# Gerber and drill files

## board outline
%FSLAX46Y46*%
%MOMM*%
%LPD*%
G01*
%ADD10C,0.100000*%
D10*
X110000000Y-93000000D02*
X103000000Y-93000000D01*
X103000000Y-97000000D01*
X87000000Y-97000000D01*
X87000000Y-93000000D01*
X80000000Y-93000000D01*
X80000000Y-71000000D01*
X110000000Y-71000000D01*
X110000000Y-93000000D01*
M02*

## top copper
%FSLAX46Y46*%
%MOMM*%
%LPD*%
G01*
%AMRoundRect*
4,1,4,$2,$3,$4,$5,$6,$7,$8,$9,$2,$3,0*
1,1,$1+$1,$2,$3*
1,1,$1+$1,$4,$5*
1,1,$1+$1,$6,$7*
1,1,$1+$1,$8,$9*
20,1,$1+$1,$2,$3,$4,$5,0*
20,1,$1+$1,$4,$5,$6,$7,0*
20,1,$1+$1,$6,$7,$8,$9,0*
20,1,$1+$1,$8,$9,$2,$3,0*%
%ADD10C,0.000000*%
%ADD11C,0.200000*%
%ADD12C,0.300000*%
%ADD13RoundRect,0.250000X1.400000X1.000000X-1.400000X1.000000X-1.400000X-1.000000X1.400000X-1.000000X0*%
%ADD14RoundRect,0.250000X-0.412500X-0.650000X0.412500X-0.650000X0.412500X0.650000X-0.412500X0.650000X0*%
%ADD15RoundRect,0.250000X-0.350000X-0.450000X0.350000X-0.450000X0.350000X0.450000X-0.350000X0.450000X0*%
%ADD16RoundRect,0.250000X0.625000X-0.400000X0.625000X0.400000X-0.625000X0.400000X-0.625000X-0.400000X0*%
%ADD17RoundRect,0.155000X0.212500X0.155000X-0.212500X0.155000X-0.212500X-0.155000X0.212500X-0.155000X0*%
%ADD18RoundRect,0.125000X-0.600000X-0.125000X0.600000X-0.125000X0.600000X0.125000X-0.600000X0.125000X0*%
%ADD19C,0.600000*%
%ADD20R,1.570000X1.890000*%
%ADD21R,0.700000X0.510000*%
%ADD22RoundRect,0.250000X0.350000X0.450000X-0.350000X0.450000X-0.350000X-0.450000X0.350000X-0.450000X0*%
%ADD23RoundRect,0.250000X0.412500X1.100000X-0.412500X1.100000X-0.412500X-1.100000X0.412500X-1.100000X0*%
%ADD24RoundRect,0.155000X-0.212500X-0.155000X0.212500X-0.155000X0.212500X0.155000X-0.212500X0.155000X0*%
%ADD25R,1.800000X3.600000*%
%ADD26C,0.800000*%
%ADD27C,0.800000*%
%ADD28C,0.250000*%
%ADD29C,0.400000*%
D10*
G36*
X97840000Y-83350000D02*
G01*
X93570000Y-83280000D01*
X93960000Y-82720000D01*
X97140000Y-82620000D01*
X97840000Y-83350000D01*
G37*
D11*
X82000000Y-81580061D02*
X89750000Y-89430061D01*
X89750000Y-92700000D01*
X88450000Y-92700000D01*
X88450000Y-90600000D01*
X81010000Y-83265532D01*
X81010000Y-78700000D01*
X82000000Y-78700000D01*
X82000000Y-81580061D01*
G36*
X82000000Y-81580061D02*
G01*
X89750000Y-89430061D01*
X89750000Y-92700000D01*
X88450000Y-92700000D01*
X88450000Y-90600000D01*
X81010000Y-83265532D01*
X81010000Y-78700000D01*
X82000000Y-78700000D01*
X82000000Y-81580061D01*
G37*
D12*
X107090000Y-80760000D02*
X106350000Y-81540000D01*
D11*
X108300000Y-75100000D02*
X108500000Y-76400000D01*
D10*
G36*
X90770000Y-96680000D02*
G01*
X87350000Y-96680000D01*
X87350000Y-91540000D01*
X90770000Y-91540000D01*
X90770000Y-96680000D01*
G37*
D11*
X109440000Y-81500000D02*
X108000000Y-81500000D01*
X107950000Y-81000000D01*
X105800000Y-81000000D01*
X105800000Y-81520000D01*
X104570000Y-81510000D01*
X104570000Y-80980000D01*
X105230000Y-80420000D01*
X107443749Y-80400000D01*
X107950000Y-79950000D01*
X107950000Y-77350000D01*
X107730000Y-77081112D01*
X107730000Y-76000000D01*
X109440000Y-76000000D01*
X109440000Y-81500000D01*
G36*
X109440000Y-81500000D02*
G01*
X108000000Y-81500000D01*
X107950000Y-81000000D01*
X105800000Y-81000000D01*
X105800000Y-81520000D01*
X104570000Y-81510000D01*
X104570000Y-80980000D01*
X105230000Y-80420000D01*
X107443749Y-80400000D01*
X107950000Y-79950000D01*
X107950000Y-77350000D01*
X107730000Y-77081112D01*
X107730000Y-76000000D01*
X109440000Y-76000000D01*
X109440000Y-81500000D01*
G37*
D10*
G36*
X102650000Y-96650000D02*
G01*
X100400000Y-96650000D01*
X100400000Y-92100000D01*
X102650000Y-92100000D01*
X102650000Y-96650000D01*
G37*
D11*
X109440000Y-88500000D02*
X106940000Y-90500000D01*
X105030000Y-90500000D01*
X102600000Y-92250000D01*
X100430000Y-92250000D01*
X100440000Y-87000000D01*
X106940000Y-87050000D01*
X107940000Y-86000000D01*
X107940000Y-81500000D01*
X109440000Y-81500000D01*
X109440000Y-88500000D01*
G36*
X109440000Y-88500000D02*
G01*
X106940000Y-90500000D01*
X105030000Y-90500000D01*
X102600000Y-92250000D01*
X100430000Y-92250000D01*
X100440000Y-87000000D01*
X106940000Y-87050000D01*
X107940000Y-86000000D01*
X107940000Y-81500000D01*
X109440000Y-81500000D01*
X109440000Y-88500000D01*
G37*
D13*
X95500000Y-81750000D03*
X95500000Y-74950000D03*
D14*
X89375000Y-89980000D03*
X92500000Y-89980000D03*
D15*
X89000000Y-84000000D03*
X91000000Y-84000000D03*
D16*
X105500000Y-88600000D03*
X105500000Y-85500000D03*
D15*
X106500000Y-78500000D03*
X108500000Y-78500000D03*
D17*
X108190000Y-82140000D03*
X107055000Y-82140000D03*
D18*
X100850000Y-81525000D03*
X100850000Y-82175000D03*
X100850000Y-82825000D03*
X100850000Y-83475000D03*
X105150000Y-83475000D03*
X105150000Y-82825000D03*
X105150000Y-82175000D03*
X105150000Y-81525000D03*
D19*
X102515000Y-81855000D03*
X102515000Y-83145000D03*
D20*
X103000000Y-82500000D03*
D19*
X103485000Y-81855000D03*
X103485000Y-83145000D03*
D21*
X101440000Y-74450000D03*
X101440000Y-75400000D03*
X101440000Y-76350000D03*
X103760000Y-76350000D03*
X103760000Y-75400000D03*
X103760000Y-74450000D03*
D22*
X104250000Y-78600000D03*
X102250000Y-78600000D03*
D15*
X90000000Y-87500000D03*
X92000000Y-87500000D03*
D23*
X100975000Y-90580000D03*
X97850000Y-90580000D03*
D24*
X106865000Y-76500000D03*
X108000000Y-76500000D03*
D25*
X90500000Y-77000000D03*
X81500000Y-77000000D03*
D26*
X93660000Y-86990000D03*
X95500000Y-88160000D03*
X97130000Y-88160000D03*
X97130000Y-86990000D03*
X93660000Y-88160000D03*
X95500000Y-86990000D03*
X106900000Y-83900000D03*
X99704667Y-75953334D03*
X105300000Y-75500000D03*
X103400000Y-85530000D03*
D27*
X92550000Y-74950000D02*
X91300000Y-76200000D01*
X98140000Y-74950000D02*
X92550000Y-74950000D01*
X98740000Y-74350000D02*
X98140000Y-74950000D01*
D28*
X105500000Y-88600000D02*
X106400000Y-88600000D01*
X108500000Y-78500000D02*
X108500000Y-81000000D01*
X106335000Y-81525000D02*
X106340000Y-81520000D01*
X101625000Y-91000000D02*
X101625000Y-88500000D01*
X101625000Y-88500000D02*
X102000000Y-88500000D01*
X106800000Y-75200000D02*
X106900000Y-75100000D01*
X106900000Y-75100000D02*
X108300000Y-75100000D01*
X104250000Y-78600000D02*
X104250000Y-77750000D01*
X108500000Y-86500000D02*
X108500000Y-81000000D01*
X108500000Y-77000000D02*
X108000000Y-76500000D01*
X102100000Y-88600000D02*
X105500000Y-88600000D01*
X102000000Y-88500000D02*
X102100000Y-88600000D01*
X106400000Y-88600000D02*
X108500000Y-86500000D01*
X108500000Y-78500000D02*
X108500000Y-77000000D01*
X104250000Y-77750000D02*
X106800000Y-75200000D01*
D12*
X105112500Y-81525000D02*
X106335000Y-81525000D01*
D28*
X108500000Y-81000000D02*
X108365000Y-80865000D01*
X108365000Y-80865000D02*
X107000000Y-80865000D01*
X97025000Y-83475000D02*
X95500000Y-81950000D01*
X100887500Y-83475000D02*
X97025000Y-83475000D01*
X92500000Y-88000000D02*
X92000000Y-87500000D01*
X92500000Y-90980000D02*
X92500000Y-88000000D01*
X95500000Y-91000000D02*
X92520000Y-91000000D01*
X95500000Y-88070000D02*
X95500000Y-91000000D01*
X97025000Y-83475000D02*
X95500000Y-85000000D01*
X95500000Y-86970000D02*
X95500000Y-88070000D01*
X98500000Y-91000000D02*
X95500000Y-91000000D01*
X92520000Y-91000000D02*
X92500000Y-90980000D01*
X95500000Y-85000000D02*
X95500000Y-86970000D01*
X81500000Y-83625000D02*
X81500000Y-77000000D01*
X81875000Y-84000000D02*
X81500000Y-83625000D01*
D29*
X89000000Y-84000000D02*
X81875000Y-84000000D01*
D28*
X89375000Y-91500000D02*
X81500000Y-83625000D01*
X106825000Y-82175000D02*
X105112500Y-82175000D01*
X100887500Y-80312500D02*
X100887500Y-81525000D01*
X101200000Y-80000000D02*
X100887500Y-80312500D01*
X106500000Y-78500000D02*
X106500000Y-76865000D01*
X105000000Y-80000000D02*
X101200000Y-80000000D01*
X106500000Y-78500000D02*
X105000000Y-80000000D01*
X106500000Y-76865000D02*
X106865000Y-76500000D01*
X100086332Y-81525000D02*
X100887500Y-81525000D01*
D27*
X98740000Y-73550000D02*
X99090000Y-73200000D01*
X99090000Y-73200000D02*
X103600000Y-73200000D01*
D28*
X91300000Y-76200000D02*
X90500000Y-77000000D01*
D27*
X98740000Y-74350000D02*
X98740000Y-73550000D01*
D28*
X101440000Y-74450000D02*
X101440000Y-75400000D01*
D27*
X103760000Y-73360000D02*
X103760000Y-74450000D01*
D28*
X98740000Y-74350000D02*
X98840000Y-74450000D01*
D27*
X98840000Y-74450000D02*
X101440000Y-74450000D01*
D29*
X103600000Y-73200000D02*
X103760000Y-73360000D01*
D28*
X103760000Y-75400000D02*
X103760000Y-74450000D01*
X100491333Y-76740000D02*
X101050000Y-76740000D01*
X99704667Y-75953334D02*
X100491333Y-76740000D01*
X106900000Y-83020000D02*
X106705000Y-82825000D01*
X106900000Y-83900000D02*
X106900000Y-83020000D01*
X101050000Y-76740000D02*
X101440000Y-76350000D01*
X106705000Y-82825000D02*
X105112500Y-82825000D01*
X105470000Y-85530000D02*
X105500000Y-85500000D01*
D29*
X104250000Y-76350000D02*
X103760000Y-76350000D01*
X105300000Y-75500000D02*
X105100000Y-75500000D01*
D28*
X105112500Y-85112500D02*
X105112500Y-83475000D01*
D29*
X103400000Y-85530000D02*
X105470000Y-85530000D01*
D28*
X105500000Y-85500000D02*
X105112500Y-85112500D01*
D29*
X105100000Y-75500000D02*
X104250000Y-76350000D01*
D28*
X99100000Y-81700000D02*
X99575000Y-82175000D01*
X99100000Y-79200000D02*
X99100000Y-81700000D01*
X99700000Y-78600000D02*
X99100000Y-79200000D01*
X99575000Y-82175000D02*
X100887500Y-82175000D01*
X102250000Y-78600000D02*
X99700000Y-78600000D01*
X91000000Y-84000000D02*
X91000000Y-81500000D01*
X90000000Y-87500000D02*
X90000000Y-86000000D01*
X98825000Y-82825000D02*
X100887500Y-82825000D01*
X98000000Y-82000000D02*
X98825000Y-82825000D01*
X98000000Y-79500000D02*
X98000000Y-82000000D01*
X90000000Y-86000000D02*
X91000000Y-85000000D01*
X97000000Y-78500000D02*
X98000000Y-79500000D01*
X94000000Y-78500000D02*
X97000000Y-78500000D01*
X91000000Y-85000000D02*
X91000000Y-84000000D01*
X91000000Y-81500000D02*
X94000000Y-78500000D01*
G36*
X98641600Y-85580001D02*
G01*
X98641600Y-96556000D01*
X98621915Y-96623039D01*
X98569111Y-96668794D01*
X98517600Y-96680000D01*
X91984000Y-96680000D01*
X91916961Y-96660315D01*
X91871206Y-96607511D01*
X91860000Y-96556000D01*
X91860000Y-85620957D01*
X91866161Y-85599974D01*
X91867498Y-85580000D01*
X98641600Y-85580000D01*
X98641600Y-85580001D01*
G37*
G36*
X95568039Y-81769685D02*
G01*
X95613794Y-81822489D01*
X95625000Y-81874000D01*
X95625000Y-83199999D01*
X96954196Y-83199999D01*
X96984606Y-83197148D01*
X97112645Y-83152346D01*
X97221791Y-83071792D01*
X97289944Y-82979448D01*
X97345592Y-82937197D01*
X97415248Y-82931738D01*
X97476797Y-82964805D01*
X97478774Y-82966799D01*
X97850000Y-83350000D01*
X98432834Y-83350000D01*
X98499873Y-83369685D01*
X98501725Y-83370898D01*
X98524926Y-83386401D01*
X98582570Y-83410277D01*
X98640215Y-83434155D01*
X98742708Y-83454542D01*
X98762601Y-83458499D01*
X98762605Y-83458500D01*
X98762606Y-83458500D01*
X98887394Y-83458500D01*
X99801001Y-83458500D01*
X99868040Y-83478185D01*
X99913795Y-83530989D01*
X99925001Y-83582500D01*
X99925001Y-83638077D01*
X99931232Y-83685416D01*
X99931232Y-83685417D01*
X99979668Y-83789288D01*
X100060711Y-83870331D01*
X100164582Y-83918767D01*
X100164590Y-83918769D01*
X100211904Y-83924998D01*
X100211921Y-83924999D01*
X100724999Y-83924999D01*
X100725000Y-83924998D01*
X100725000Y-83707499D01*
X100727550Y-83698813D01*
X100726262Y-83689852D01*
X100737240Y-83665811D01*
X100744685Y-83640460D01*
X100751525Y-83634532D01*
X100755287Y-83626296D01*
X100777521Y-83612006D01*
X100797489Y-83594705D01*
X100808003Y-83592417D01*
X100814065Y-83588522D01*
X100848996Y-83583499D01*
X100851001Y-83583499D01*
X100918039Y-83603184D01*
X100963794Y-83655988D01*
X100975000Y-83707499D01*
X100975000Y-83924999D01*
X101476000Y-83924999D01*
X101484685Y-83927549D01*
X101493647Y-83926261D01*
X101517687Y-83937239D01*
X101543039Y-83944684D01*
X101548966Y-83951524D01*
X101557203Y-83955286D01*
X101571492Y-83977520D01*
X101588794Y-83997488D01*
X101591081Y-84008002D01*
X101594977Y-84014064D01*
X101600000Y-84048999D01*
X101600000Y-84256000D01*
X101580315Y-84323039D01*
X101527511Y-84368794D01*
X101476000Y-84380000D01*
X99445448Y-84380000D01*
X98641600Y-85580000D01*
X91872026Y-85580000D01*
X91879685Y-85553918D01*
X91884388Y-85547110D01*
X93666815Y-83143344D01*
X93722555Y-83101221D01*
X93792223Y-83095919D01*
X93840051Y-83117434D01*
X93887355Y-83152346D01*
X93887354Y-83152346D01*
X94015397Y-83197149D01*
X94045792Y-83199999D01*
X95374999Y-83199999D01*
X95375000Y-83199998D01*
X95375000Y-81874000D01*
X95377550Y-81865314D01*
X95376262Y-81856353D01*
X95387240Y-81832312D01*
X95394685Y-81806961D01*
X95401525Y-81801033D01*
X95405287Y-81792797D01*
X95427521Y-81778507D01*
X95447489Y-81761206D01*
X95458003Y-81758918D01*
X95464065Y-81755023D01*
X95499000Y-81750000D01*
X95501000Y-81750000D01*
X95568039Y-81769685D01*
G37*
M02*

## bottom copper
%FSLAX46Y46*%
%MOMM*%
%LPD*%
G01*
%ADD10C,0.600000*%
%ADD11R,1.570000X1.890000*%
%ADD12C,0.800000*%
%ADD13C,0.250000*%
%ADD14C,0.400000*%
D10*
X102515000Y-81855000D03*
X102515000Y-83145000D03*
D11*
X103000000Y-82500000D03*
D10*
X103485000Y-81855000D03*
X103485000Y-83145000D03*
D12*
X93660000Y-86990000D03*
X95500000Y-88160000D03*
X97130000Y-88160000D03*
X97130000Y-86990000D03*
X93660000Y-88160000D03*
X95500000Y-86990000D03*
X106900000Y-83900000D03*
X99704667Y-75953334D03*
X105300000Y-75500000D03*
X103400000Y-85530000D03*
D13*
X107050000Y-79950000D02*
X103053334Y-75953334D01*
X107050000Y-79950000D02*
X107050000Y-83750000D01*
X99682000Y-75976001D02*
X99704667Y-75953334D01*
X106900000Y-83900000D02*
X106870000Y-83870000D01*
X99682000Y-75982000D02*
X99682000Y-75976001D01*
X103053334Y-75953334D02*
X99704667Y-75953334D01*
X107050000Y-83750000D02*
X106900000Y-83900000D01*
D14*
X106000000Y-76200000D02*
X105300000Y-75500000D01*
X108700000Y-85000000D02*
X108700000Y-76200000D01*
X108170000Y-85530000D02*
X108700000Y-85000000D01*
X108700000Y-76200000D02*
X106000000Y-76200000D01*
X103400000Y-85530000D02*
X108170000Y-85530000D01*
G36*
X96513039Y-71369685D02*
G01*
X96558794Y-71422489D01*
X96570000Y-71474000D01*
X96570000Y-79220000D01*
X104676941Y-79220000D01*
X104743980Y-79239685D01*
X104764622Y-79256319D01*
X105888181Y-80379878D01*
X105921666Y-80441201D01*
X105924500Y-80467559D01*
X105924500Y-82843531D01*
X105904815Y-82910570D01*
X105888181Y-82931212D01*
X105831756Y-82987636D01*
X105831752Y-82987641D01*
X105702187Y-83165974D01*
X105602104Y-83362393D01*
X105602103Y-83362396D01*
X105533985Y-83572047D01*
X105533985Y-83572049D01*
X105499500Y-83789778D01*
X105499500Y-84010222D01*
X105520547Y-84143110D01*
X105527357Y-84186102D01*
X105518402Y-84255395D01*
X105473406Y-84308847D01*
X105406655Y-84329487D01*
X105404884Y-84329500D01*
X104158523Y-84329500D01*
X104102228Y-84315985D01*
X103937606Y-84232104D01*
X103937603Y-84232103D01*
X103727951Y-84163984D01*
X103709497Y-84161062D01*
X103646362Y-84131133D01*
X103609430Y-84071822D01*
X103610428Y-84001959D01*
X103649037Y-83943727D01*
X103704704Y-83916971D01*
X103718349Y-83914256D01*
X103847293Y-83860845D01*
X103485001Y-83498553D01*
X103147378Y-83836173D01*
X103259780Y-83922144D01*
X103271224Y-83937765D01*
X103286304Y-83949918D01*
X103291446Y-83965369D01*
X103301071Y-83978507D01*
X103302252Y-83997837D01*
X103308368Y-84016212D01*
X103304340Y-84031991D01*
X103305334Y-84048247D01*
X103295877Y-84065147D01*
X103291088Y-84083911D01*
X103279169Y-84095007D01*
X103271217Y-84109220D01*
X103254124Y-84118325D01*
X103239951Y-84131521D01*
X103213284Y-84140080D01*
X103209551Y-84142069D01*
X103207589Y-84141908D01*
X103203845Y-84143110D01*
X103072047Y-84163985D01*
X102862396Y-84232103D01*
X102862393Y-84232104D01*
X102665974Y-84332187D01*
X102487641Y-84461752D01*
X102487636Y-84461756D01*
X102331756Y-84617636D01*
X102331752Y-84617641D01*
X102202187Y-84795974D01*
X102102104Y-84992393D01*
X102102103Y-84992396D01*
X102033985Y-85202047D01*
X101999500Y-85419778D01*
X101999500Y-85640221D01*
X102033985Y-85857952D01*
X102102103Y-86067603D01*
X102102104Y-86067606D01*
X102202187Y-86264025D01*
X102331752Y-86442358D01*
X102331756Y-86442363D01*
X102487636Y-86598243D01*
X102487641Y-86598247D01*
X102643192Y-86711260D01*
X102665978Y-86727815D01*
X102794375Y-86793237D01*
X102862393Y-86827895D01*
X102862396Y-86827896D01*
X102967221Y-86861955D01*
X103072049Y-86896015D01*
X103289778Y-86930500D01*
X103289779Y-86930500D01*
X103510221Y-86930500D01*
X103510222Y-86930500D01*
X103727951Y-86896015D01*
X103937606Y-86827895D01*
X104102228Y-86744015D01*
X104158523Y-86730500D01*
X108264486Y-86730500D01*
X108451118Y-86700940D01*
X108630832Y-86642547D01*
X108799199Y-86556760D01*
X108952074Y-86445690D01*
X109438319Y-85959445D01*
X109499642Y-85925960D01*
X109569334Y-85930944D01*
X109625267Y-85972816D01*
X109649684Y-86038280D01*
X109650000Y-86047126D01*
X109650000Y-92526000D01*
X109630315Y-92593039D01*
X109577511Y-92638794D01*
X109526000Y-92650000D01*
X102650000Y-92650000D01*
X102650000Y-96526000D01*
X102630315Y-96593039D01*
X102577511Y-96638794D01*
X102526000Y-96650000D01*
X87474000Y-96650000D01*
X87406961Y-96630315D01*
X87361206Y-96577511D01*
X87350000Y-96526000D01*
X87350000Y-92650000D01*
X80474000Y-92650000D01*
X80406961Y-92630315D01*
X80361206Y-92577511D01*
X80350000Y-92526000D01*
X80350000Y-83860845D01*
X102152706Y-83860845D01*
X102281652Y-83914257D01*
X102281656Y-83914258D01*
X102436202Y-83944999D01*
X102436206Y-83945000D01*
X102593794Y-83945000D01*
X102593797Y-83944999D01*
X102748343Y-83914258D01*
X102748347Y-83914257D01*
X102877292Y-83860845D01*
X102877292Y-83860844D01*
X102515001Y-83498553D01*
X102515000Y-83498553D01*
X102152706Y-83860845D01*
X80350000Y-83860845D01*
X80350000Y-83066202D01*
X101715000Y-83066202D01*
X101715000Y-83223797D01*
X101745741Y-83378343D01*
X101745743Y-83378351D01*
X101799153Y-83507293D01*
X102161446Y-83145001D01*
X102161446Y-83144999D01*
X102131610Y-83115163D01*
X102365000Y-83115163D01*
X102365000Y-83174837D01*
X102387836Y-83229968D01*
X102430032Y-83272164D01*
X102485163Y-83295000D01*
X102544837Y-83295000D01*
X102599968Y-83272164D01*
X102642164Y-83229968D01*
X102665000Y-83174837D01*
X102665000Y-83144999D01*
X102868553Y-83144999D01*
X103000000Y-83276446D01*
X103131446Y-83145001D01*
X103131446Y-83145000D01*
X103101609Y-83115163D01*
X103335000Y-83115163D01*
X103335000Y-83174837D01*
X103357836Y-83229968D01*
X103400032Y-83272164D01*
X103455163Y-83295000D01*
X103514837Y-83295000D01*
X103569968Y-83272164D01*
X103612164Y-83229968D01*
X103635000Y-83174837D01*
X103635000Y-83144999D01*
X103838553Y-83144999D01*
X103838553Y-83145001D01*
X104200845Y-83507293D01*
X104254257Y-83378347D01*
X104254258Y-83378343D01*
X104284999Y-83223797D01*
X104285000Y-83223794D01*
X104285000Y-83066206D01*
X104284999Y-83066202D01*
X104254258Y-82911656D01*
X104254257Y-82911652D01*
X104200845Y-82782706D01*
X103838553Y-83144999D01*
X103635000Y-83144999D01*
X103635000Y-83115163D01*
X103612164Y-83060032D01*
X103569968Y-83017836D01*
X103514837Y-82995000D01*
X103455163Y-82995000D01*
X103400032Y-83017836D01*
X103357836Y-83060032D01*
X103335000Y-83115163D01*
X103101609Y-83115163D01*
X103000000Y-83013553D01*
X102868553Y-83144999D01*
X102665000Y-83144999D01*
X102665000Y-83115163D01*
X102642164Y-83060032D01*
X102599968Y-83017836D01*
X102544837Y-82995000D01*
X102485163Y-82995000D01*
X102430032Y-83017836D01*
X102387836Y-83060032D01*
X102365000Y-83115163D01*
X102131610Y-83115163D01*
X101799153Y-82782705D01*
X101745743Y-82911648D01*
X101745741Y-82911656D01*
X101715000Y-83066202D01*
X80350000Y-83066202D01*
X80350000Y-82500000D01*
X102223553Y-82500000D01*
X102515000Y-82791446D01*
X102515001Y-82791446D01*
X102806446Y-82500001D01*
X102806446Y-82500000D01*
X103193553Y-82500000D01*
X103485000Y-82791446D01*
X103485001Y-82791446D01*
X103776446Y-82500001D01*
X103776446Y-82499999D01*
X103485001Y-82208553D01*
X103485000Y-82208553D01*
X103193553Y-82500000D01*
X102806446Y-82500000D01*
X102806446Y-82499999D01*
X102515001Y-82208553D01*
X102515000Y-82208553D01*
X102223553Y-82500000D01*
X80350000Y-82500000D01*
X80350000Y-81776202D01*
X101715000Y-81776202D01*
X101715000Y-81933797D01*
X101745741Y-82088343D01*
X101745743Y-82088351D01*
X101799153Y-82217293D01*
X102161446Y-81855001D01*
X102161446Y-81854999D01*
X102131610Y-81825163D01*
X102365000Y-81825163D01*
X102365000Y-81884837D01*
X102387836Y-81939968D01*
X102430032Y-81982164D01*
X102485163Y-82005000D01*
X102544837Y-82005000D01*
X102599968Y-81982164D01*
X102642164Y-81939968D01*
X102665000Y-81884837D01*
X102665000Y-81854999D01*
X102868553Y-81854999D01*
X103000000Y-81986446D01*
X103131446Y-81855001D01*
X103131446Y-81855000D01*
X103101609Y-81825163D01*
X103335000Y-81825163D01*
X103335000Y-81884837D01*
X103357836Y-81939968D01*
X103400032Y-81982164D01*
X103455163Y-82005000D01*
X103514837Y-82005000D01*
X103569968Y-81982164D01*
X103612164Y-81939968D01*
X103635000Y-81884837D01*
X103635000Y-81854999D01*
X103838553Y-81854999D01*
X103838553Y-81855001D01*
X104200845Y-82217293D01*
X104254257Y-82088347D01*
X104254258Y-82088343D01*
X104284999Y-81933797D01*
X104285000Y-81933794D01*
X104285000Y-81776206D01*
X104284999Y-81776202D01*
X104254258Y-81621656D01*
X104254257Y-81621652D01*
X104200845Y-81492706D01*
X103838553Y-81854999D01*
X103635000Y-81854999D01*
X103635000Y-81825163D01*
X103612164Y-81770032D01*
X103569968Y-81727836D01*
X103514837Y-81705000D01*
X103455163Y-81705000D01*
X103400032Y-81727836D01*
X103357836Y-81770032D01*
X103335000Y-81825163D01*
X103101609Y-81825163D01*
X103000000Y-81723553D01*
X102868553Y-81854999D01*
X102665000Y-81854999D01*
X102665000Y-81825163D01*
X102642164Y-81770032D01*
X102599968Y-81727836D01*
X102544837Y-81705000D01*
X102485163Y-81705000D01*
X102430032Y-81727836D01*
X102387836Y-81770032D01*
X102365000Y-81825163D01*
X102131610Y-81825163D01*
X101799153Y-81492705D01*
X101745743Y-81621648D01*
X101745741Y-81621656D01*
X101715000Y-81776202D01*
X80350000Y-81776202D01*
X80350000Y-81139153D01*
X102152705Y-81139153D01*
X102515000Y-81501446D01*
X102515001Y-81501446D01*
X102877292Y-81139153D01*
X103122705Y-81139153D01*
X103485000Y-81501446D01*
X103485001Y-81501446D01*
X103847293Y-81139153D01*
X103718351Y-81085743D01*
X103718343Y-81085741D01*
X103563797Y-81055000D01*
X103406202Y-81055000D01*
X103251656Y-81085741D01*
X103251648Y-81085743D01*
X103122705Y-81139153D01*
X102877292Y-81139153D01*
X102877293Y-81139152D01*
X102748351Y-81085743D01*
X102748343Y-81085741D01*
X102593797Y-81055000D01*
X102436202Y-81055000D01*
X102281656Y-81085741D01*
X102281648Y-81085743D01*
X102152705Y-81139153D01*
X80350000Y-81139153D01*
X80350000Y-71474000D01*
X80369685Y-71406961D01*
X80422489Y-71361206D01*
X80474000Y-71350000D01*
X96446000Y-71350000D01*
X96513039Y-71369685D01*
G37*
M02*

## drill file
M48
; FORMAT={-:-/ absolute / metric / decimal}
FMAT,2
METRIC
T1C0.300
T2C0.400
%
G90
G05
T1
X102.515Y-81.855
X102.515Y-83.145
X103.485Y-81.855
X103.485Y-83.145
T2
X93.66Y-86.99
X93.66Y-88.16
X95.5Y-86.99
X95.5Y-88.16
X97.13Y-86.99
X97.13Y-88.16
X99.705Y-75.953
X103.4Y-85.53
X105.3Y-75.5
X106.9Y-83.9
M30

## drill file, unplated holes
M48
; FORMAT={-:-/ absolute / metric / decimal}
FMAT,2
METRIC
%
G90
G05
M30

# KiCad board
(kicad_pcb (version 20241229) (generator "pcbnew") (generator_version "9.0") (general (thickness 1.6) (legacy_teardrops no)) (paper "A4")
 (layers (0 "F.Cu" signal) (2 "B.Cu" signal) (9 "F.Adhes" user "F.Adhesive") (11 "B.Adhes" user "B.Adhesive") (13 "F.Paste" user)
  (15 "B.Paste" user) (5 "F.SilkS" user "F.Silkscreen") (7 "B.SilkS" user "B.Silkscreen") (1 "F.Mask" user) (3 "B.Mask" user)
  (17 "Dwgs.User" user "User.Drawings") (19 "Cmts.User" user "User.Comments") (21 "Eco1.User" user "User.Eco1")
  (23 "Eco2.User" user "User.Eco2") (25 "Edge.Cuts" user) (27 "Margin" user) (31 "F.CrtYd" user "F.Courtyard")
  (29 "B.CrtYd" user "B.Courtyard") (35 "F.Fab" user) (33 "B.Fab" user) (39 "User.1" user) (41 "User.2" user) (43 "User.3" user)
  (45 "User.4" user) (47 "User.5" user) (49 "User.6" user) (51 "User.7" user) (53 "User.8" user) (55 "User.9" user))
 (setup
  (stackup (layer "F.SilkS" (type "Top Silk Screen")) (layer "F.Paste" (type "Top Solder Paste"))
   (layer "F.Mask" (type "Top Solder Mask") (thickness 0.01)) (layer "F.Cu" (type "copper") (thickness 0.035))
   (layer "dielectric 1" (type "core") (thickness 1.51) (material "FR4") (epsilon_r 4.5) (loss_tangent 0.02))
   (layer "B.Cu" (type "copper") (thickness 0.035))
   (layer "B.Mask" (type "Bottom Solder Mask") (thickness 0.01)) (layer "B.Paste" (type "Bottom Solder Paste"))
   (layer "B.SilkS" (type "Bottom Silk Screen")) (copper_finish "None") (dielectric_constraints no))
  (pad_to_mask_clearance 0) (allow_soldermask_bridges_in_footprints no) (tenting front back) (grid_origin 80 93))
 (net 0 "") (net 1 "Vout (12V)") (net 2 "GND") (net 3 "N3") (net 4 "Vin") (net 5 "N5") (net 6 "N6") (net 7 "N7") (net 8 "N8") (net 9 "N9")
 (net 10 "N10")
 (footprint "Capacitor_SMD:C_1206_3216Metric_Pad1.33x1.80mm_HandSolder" (layer "F.Cu") (at 90.9375 89.98)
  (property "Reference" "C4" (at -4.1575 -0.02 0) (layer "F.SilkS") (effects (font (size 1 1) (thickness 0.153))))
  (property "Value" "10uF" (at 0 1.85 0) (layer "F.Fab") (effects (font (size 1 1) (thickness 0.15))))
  (pad "1" smd roundrect (at -1.5625 0) (size 1.325 1.8) (layers "F.Cu" "F.Mask" "F.Paste") (roundrect_rratio 0.188679) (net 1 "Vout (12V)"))
  (pad "2" smd roundrect (at 1.5625 0) (size 1.325 1.8) (layers "F.Cu" "F.Mask" "F.Paste") (roundrect_rratio 0.188679) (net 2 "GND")))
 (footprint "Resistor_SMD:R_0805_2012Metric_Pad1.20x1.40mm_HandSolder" (layer "F.Cu") (at 90 84)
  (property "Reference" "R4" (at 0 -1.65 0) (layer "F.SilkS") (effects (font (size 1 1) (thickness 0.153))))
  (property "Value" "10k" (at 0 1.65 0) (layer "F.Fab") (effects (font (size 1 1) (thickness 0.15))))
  (pad "1" smd roundrect (at -1 0) (size 1.2 1.4) (layers "F.Cu" "F.Mask" "F.Paste") (roundrect_rratio 0.208333) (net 1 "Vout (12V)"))
  (pad "2" smd roundrect (at 1 0) (size 1.2 1.4) (layers "F.Cu" "F.Mask" "F.Paste") (roundrect_rratio 0.208333) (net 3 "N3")))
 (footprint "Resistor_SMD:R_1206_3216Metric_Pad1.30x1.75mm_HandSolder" (layer "F.Cu") (at 105.5 87.05 90)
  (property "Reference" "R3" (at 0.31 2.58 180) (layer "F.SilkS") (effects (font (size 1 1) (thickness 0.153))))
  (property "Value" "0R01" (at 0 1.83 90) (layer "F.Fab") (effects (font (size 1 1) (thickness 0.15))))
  (pad "1" smd roundrect (at -1.55 0 90) (size 1.3 1.75) (layers "F.Cu" "F.Mask" "F.Paste") (roundrect_rratio 0.192308) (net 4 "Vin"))
  (pad "2" smd roundrect (at 1.55 0 90) (size 1.3 1.75) (layers "F.Cu" "F.Mask" "F.Paste") (roundrect_rratio 0.192308) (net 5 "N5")))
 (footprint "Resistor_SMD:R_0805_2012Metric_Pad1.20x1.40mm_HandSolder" (layer "F.Cu") (at 107.5 78.5)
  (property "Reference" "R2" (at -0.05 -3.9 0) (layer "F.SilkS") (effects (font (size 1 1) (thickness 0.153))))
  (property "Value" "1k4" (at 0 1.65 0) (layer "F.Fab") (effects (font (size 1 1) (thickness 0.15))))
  (pad "1" smd roundrect (at -1 0) (size 1.2 1.4) (layers "F.Cu" "F.Mask" "F.Paste") (roundrect_rratio 0.208333) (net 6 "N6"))
  (pad "2" smd roundrect (at 1 0) (size 1.2 1.4) (layers "F.Cu" "F.Mask" "F.Paste") (roundrect_rratio 0.208333) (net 4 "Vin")))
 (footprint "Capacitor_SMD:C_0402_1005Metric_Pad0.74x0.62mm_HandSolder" (layer "F.Cu") (at 107.6225 82.14 180)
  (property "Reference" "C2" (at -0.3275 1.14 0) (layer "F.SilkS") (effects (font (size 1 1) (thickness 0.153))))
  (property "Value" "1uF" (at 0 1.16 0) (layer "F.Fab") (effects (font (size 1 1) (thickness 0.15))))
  (pad "1" smd roundrect (at -0.5675 0 180) (size 0.735 0.62) (layers "F.Cu" "F.Mask" "F.Paste") (roundrect_rratio 0.25) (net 4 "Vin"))
  (pad "2" smd roundrect (at 0.5675 0 180) (size 0.735 0.62) (layers "F.Cu" "F.Mask" "F.Paste") (roundrect_rratio 0.25) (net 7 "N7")))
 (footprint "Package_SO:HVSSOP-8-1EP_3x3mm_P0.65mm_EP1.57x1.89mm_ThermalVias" (layer "F.Cu") (at 103 82.5)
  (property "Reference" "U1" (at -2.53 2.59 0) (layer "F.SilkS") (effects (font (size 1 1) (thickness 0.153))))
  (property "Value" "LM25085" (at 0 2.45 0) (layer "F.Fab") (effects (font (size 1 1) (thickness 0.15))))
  (pad "" smd roundrect (at -0.39 -0.47) (size 0.63 0.76) (layers "F.Paste") (roundrect_rratio 0.25))
  (pad "" smd roundrect (at -0.39 0.47) (size 0.63 0.76) (layers "F.Paste") (roundrect_rratio 0.25))
  (pad "" smd roundrect (at 0.39 -0.47) (size 0.63 0.76) (layers "F.Paste") (roundrect_rratio 0.25))
  (pad "" smd roundrect (at 0.39 0.47) (size 0.63 0.76) (layers "F.Paste") (roundrect_rratio 0.25))
  (pad "1" smd roundrect (at -2.15 -0.975) (size 1.45 0.5) (layers "F.Cu" "F.Mask" "F.Paste") (roundrect_rratio 0.25) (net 6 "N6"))
  (pad "2" smd roundrect (at -2.15 -0.325) (size 1.45 0.5) (layers "F.Cu" "F.Mask" "F.Paste") (roundrect_rratio 0.25) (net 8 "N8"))
  (pad "3" smd roundrect (at -2.15 0.325) (size 1.45 0.5) (layers "F.Cu" "F.Mask" "F.Paste") (roundrect_rratio 0.25) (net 3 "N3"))
  (pad "4" smd roundrect (at -2.15 0.975) (size 1.45 0.5) (layers "F.Cu" "F.Mask" "F.Paste") (roundrect_rratio 0.25) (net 2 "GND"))
  (pad "5" smd roundrect (at 2.15 0.975) (size 1.45 0.5) (layers "F.Cu" "F.Mask" "F.Paste") (roundrect_rratio 0.25) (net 5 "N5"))
  (pad "6" smd roundrect (at 2.15 0.325) (size 1.45 0.5) (layers "F.Cu" "F.Mask" "F.Paste") (roundrect_rratio 0.25) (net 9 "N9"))
  (pad "7" smd roundrect (at 2.15 -0.325) (size 1.45 0.5) (layers "F.Cu" "F.Mask" "F.Paste") (roundrect_rratio 0.25) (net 7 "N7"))
  (pad "8" smd roundrect (at 2.15 -0.975) (size 1.45 0.5) (layers "F.Cu" "F.Mask" "F.Paste") (roundrect_rratio 0.25) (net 4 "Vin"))
  (pad "9" thru_hole circle (at -0.485 -0.645) (size 0.6 0.6) (drill 0.3) (layers "*.Cu") (remove_unused_layers no) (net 2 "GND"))
  (pad "9" thru_hole circle (at -0.485 0.645) (size 0.6 0.6) (drill 0.3) (layers "*.Cu") (remove_unused_layers no) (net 2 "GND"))
  (pad "9" smd rect (at 0 0) (size 1.57 1.89) (layers "F.Cu" "F.Mask") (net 2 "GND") (zone_connect 2))
  (pad "9" smd rect (at 0 0) (size 1.57 1.89) (layers "B.Cu") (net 2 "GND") (zone_connect 2))
  (pad "9" thru_hole circle (at 0.485 -0.645) (size 0.6 0.6) (drill 0.3) (layers "*.Cu") (remove_unused_layers no) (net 2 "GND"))
  (pad "9" thru_hole circle (at 0.485 0.645) (size 0.6 0.6) (drill 0.3) (layers "*.Cu") (remove_unused_layers no) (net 2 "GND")))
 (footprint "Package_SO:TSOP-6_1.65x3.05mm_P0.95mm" (layer "F.Cu") (at 102.6 75.4)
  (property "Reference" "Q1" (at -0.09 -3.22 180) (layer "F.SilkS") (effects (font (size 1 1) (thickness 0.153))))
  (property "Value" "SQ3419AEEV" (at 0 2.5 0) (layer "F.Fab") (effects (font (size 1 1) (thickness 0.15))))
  (pad "1" smd rect (at -1.16 -0.95) (size 0.7 0.51) (layers "F.Cu" "F.Mask" "F.Paste") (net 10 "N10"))
  (pad "2" smd rect (at -1.16 0) (size 0.7 0.51) (layers "F.Cu" "F.Mask" "F.Paste") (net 10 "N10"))
  (pad "3" smd rect (at -1.16 0.95) (size 0.7 0.51) (layers "F.Cu" "F.Mask" "F.Paste") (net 9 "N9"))
  (pad "4" smd rect (at 1.16 0.95) (size 0.7 0.51) (layers "F.Cu" "F.Mask" "F.Paste") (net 5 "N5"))
  (pad "5" smd rect (at 1.16 0) (size 0.7 0.51) (layers "F.Cu" "F.Mask" "F.Paste") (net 10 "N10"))
  (pad "6" smd rect (at 1.16 -0.95) (size 0.7 0.51) (layers "F.Cu" "F.Mask" "F.Paste") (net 10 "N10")))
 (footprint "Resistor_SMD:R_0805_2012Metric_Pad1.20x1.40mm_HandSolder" (layer "F.Cu") (at 103.25 78.6 180)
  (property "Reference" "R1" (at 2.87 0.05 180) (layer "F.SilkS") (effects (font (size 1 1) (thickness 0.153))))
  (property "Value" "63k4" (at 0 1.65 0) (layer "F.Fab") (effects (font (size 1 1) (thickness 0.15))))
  (pad "1" smd roundrect (at -1 0 180) (size 1.2 1.4) (layers "F.Cu" "F.Mask" "F.Paste") (roundrect_rratio 0.208333) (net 4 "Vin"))
  (pad "2" smd roundrect (at 1 0 180) (size 1.2 1.4) (layers "F.Cu" "F.Mask" "F.Paste") (roundrect_rratio 0.208333) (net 8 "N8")))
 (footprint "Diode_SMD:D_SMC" (layer "F.Cu") (at 95.5 78.35 90)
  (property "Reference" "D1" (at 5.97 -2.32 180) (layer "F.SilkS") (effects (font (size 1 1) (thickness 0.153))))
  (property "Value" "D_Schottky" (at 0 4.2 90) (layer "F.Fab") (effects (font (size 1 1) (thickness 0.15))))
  (pad "1" smd roundrect (at -3.4 0 180) (size 3.3 2.5) (layers "F.Cu" "F.Mask" "F.Paste") (roundrect_rratio 0.1) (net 2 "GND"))
  (pad "2" smd roundrect (at 3.4 0 180) (size 3.3 2.5) (layers "F.Cu" "F.Mask" "F.Paste") (roundrect_rratio 0.1) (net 10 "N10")))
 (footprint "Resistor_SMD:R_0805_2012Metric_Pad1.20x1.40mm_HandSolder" (layer "F.Cu") (at 91 87.5)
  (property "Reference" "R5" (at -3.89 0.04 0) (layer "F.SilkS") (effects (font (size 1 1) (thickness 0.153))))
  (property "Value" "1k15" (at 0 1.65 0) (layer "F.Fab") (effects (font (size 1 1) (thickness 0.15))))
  (pad "1" smd roundrect (at -1 0) (size 1.2 1.4) (layers "F.Cu" "F.Mask" "F.Paste") (roundrect_rratio 0.208333) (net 3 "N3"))
  (pad "2" smd roundrect (at 1 0) (size 1.2 1.4) (layers "F.Cu" "F.Mask" "F.Paste") (roundrect_rratio 0.208333) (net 2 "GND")))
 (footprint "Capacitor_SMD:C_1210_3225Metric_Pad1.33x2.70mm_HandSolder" (layer "F.Cu") (at 99.4125 90.58 180)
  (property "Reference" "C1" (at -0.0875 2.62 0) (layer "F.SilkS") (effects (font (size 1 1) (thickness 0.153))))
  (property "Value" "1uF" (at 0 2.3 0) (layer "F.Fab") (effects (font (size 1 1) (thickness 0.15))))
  (pad "1" smd roundrect (at -1.5625 0 180) (size 1.325 2.7) (layers "F.Cu" "F.Mask" "F.Paste") (roundrect_rratio 0.188679) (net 4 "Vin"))
  (pad "2" smd roundrect (at 1.5625 0 180) (size 1.325 2.7) (layers "F.Cu" "F.Mask" "F.Paste") (roundrect_rratio 0.188679) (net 2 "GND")))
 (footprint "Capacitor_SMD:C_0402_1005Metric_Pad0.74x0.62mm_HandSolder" (layer "F.Cu") (at 107.4325 76.5)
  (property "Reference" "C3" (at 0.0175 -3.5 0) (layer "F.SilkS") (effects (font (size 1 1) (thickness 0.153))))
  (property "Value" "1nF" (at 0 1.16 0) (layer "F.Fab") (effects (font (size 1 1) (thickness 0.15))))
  (pad "1" smd roundrect (at -0.5675 0) (size 0.735 0.62) (layers "F.Cu" "F.Mask" "F.Paste") (roundrect_rratio 0.25) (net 6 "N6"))
  (pad "2" smd roundrect (at 0.5675 0) (size 0.735 0.62) (layers "F.Cu" "F.Mask" "F.Paste") (roundrect_rratio 0.25) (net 4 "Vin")))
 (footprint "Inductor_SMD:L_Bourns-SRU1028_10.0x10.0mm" (layer "F.Cu") (at 86 77 180)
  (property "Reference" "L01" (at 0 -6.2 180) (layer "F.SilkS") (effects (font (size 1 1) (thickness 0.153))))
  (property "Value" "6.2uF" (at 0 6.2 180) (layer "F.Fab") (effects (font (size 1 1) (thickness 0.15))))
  (pad "1" smd rect (at -4.5 0 180) (size 1.8 3.6) (layers "F.Cu" "F.Mask" "F.Paste") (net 10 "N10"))
  (pad "2" smd rect (at 4.5 0 180) (size 1.8 3.6) (layers "F.Cu" "F.Mask" "F.Paste") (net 1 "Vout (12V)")))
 (gr_poly
  (pts (xy 89.75 89.430061) (xy 82 81.580061) (xy 82 78.7) (xy 81.01 78.7) (xy 81.01 83.265532) (xy 88.45 90.6) (xy 88.45 92.7)
   (xy 89.75 92.7))
  (stroke (width 0.2) (type solid)) (fill yes) (layer "F.Cu") (net 1))
 (gr_line (start 107.09 80.76) (end 106.35 81.54) (stroke (width 0.3) (type solid)) (layer "F.Cu") (net 4))
 (gr_line (start 108.3 75.1) (end 108.5 76.4) (stroke (width 0.2) (type default)) (layer "F.Cu") (net 4))
 (gr_poly
  (pts (xy 87.35 96.68) (xy 87.35 91.54) (xy 90.77 91.54) (xy 90.77 96.68)) (stroke (width 0) (type solid)) (fill yes) (layer "F.Cu")
  (net 1))
 (gr_poly
  (pts (xy 109.44 81.5) (xy 109.44 76) (xy 107.73 76) (xy 107.73 77.081112) (xy 107.95 77.35) (xy 107.95 79.95) (xy 107.443749 80.4)
   (xy 105.23 80.42) (xy 104.57 80.98) (xy 104.57 81.51) (xy 105.8 81.52) (xy 105.8 81) (xy 107.95 81) (xy 108 81.5))
  (stroke (width 0.2) (type solid)) (fill yes) (layer "F.Cu") (net 4))
 (gr_poly
  (pts (xy 102.65 96.65) (xy 102.65 92.1) (xy 100.4 92.1) (xy 100.4 96.65)) (stroke (width 0) (type solid)) (fill yes) (layer "F.Cu")
  (net 4))
 (gr_poly
  (pts (xy 97.14 82.62) (xy 97.84 83.35) (xy 93.57 83.28) (xy 93.96 82.72)) (stroke (width 0) (type solid)) (fill yes) (layer "F.Cu")
  (net 2))
 (gr_poly
  (pts (xy 100.43 92.25) (xy 100.44 87) (xy 106.94 87.05) (xy 107.94 86) (xy 107.94 81.5) (xy 109.44 81.5) (xy 109.44 88.5) (xy 106.94 90.5)
   (xy 105.03 90.5) (xy 102.6 92.25))
  (stroke (width 0.2) (type solid)) (fill yes) (layer "F.Cu") (net 4))
 (gr_poly
  (pts (xy 110 93) (xy 103 93) (xy 103 97) (xy 87 97) (xy 87 93) (xy 80 93) (xy 80 71) (xy 110 71)) (stroke (width 0.1) (type solid))
  (fill no) (layer "Edge.Cuts"))
 (segment (start 105.5 88.6) (end 106.4 88.6) (width 0.25) (layer "F.Cu") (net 4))
 (segment (start 108.5 78.5) (end 108.5 81) (width 0.25) (layer "F.Cu") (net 4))
 (segment (start 106.335 81.525) (end 106.34 81.52) (width 0.25) (layer "F.Cu") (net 4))
 (segment (start 101.625 91) (end 101.625 88.5) (width 0.25) (layer "F.Cu") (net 4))
 (segment (start 101.625 88.5) (end 102 88.5) (width 0.25) (layer "F.Cu") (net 4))
 (segment (start 106.8 75.2) (end 106.9 75.1) (width 0.25) (layer "F.Cu") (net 4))
 (segment (start 106.9 75.1) (end 108.3 75.1) (width 0.25) (layer "F.Cu") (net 4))
 (segment (start 104.25 78.6) (end 104.25 77.75) (width 0.25) (layer "F.Cu") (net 4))
 (segment (start 108.5 86.5) (end 108.5 81) (width 0.25) (layer "F.Cu") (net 4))
 (segment (start 108.5 77) (end 108 76.5) (width 0.25) (layer "F.Cu") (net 4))
 (segment (start 102.1 88.6) (end 105.5 88.6) (width 0.25) (layer "F.Cu") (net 4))
 (segment (start 102 88.5) (end 102.1 88.6) (width 0.25) (layer "F.Cu") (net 4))
 (segment (start 106.4 88.6) (end 108.5 86.5) (width 0.25) (layer "F.Cu") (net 4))
 (segment (start 108.5 78.5) (end 108.5 77) (width 0.25) (layer "F.Cu") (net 4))
 (segment (start 104.25 77.75) (end 106.8 75.2) (width 0.25) (layer "F.Cu") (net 4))
 (segment (start 105.1125 81.525) (end 106.335 81.525) (width 0.3) (layer "F.Cu") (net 4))
 (segment (start 108.5 81) (end 108.365 80.865) (width 0.25) (layer "F.Cu") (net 4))
 (segment (start 108.365 80.865) (end 107 80.865) (width 0.25) (layer "F.Cu") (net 4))
 (segment (start 97.025 83.475) (end 95.5 81.95) (width 0.25) (layer "F.Cu") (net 2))
 (segment (start 100.8875 83.475) (end 97.025 83.475) (width 0.25) (layer "F.Cu") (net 2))
 (segment (start 92.5 88) (end 92 87.5) (width 0.25) (layer "F.Cu") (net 2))
 (segment (start 92.5 90.98) (end 92.5 88) (width 0.25) (layer "F.Cu") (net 2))
 (segment (start 95.5 91) (end 92.52 91) (width 0.25) (layer "F.Cu") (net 2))
 (segment (start 95.5 88.07) (end 95.5 91) (width 0.25) (layer "F.Cu") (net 2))
 (segment (start 97.025 83.475) (end 95.5 85) (width 0.25) (layer "F.Cu") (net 2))
 (segment (start 95.5 86.97) (end 95.5 88.07) (width 0.25) (layer "F.Cu") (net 2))
 (segment (start 98.5 91) (end 95.5 91) (width 0.25) (layer "F.Cu") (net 2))
 (segment (start 92.52 91) (end 92.5 90.98) (width 0.25) (layer "F.Cu") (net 2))
 (segment (start 95.5 85) (end 95.5 86.97) (width 0.25) (layer "F.Cu") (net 2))
 (via (at 93.66 86.99) (size 0.8) (drill 0.4) (layers "F.Cu" "B.Cu") (free yes) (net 2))
 (via (at 95.5 88.16) (size 0.8) (drill 0.4) (layers "F.Cu" "B.Cu") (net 2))
 (via (at 97.13 88.16) (size 0.8) (drill 0.4) (layers "F.Cu" "B.Cu") (free yes) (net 2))
 (via (at 97.13 86.99) (size 0.8) (drill 0.4) (layers "F.Cu" "B.Cu") (free yes) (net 2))
 (via (at 93.66 88.16) (size 0.8) (drill 0.4) (layers "F.Cu" "B.Cu") (free yes) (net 2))
 (via (at 95.5 86.99) (size 0.8) (drill 0.4) (layers "F.Cu" "B.Cu") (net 2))
 (segment (start 81.5 83.625) (end 81.5 77) (width 0.25) (layer "F.Cu") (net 1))
 (segment (start 81.875 84) (end 81.5 83.625) (width 0.25) (layer "F.Cu") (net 1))
 (segment (start 89 84) (end 81.875 84) (width 0.4) (layer "F.Cu") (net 1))
 (segment (start 89.375 91.5) (end 81.5 83.625) (width 0.25) (layer "F.Cu") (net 1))
 (segment (start 106.825 82.175) (end 105.1125 82.175) (width 0.25) (layer "F.Cu") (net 7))
 (segment (start 100.8875 80.3125) (end 100.8875 81.525) (width 0.25) (layer "F.Cu") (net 6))
 (segment (start 101.2 80) (end 100.8875 80.3125) (width 0.25) (layer "F.Cu") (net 6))
 (segment (start 106.5 78.5) (end 106.5 76.865) (width 0.25) (layer "F.Cu") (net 6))
 (segment (start 105 80) (end 101.2 80) (width 0.25) (layer "F.Cu") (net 6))
 (segment (start 106.5 78.5) (end 105 80) (width 0.25) (layer "F.Cu") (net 6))
 (segment (start 106.5 76.865) (end 106.865 76.5) (width 0.25) (layer "F.Cu") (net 6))
 (segment (start 100.086332 81.525) (end 100.8875 81.525) (width 0.25) (layer "F.Cu") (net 6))
 (segment (start 98.74 73.55) (end 99.09 73.2) (width 0.8) (layer "F.Cu") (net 10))
 (segment (start 99.09 73.2) (end 103.6 73.2) (width 0.8) (layer "F.Cu") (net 10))
 (segment (start 91.3 76.2) (end 90.5 77) (width 0.25) (layer "F.Cu") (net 10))
 (segment (start 98.74 74.35) (end 98.14 74.95) (width 0.8) (layer "F.Cu") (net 10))
 (segment (start 98.14 74.95) (end 92.55 74.95) (width 0.8) (layer "F.Cu") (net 10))
 (segment (start 98.74 74.35) (end 98.74 73.55) (width 0.8) (layer "F.Cu") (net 10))
 (segment (start 101.44 74.45) (end 101.44 75.4) (width 0.25) (layer "F.Cu") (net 10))
 (segment (start 103.76 73.36) (end 103.76 74.45) (width 0.8) (layer "F.Cu") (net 10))
 (segment (start 92.55 74.95) (end 91.3 76.2) (width 0.8) (layer "F.Cu") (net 10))
 (segment (start 98.74 74.35) (end 98.84 74.45) (width 0.25) (layer "F.Cu") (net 10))
 (segment (start 98.84 74.45) (end 101.44 74.45) (width 0.8) (layer "F.Cu") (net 10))
 (segment (start 103.6 73.2) (end 103.76 73.36) (width 0.4) (layer "F.Cu") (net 10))
 (segment (start 103.76 75.4) (end 103.76 74.45) (width 0.25) (layer "F.Cu") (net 10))
 (segment (start 100.491333 76.74) (end 101.05 76.74) (width 0.25) (layer "F.Cu") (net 9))
 (segment (start 99.704667 75.953334) (end 100.491333 76.74) (width 0.25) (layer "F.Cu") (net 9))
 (segment (start 106.9 83.02) (end 106.705 82.825) (width 0.25) (layer "F.Cu") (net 9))
 (segment (start 106.9 83.9) (end 106.9 83.02) (width 0.25) (layer "F.Cu") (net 9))
 (segment (start 101.05 76.74) (end 101.44 76.35) (width 0.25) (layer "F.Cu") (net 9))
 (segment (start 106.705 82.825) (end 105.1125 82.825) (width 0.25) (layer "F.Cu") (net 9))
 (via (at 106.9 83.9) (size 0.8) (drill 0.4) (layers "F.Cu" "B.Cu") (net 9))
 (via (at 99.704667 75.953334) (size 0.8) (drill 0.4) (layers "F.Cu" "B.Cu") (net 9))
 (segment (start 107.05 79.95) (end 103.053334 75.953334) (width 0.25) (layer "B.Cu") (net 9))
 (segment (start 107.05 79.95) (end 107.05 83.75) (width 0.25) (layer "B.Cu") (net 9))
 (segment (start 99.682 75.976001) (end 99.704667 75.953334) (width 0.25) (layer "B.Cu") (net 9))
 (segment (start 106.9 83.9) (end 106.87 83.87) (width 0.25) (layer "B.Cu") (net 9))
 (segment (start 99.682 75.982) (end 99.682 75.976001) (width 0.25) (layer "B.Cu") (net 9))
 (segment (start 103.053334 75.953334) (end 99.704667 75.953334) (width 0.25) (layer "B.Cu") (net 9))
 (segment (start 107.05 83.75) (end 106.9 83.9) (width 0.25) (layer "B.Cu") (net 9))
 (segment (start 105.47 85.53) (end 105.5 85.5) (width 0.25) (layer "F.Cu") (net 5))
 (segment (start 104.25 76.35) (end 103.76 76.35) (width 0.4) (layer "F.Cu") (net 5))
 (segment (start 105.3 75.5) (end 105.1 75.5) (width 0.4) (layer "F.Cu") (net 5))
 (segment (start 105.1125 85.1125) (end 105.1125 83.475) (width 0.25) (layer "F.Cu") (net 5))
 (segment (start 103.4 85.53) (end 105.47 85.53) (width 0.4) (layer "F.Cu") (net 5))
 (segment (start 105.5 85.5) (end 105.1125 85.1125) (width 0.25) (layer "F.Cu") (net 5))
 (segment (start 105.1 75.5) (end 104.25 76.35) (width 0.4) (layer "F.Cu") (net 5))
 (via (at 105.3 75.5) (size 0.8) (drill 0.4) (layers "F.Cu" "B.Cu") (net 5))
 (via (at 103.4 85.53) (size 0.8) (drill 0.4) (layers "F.Cu" "B.Cu") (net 5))
 (segment (start 106 76.2) (end 105.3 75.5) (width 0.4) (layer "B.Cu") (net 5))
 (segment (start 108.7 85) (end 108.7 76.2) (width 0.4) (layer "B.Cu") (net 5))
 (segment (start 108.17 85.53) (end 108.7 85) (width 0.4) (layer "B.Cu") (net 5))
 (segment (start 108.7 76.2) (end 106 76.2) (width 0.4) (layer "B.Cu") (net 5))
 (segment (start 103.4 85.53) (end 108.17 85.53) (width 0.4) (layer "B.Cu") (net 5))
 (segment (start 99.1 81.7) (end 99.575 82.175) (width 0.25) (layer "F.Cu") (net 8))
 (segment (start 99.1 79.2) (end 99.1 81.7) (width 0.25) (layer "F.Cu") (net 8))
 (segment (start 99.7 78.6) (end 99.1 79.2) (width 0.25) (layer "F.Cu") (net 8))
 (segment (start 99.575 82.175) (end 100.8875 82.175) (width 0.25) (layer "F.Cu") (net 8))
 (segment (start 102.25 78.6) (end 99.7 78.6) (width 0.25) (layer "F.Cu") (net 8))
 (segment (start 91 84) (end 91 81.5) (width 0.25) (layer "F.Cu") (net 3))
 (segment (start 90 87.5) (end 90 86) (width 0.25) (layer "F.Cu") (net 3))
 (segment (start 98.825 82.825) (end 100.8875 82.825) (width 0.25) (layer "F.Cu") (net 3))
 (segment (start 98 82) (end 98.825 82.825) (width 0.25) (layer "F.Cu") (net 3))
 (segment (start 98 79.5) (end 98 82) (width 0.25) (layer "F.Cu") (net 3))
 (segment (start 90 86) (end 91 85) (width 0.25) (layer "F.Cu") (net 3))
 (segment (start 97 78.5) (end 98 79.5) (width 0.25) (layer "F.Cu") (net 3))
 (segment (start 94 78.5) (end 97 78.5) (width 0.25) (layer "F.Cu") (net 3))
 (segment (start 91 85) (end 91 84) (width 0.25) (layer "F.Cu") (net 3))
 (segment (start 91 81.5) (end 94 78.5) (width 0.25) (layer "F.Cu") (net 3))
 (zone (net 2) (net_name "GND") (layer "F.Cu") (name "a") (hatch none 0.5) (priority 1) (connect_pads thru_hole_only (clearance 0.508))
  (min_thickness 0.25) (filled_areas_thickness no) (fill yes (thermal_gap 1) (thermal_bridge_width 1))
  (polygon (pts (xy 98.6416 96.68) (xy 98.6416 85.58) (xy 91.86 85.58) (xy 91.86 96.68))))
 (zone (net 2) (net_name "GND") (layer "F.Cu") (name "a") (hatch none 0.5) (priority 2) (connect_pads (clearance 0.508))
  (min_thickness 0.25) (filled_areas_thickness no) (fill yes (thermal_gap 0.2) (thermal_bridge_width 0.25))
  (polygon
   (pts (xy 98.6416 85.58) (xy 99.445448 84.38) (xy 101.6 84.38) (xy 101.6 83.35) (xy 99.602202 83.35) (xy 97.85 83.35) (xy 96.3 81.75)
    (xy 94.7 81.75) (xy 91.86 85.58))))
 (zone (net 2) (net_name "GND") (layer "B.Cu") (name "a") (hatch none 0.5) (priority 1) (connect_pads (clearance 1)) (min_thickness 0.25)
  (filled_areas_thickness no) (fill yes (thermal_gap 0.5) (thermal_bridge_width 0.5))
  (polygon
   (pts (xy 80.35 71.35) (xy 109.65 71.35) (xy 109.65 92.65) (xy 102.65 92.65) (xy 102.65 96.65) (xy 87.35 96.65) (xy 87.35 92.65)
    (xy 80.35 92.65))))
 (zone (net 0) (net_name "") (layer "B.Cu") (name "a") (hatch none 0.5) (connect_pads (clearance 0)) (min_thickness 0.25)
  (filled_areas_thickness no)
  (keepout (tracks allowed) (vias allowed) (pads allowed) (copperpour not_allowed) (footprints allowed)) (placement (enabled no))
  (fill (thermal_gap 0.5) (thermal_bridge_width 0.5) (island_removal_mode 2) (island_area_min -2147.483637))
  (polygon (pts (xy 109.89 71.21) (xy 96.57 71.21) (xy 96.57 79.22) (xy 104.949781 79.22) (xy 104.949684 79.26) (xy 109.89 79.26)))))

